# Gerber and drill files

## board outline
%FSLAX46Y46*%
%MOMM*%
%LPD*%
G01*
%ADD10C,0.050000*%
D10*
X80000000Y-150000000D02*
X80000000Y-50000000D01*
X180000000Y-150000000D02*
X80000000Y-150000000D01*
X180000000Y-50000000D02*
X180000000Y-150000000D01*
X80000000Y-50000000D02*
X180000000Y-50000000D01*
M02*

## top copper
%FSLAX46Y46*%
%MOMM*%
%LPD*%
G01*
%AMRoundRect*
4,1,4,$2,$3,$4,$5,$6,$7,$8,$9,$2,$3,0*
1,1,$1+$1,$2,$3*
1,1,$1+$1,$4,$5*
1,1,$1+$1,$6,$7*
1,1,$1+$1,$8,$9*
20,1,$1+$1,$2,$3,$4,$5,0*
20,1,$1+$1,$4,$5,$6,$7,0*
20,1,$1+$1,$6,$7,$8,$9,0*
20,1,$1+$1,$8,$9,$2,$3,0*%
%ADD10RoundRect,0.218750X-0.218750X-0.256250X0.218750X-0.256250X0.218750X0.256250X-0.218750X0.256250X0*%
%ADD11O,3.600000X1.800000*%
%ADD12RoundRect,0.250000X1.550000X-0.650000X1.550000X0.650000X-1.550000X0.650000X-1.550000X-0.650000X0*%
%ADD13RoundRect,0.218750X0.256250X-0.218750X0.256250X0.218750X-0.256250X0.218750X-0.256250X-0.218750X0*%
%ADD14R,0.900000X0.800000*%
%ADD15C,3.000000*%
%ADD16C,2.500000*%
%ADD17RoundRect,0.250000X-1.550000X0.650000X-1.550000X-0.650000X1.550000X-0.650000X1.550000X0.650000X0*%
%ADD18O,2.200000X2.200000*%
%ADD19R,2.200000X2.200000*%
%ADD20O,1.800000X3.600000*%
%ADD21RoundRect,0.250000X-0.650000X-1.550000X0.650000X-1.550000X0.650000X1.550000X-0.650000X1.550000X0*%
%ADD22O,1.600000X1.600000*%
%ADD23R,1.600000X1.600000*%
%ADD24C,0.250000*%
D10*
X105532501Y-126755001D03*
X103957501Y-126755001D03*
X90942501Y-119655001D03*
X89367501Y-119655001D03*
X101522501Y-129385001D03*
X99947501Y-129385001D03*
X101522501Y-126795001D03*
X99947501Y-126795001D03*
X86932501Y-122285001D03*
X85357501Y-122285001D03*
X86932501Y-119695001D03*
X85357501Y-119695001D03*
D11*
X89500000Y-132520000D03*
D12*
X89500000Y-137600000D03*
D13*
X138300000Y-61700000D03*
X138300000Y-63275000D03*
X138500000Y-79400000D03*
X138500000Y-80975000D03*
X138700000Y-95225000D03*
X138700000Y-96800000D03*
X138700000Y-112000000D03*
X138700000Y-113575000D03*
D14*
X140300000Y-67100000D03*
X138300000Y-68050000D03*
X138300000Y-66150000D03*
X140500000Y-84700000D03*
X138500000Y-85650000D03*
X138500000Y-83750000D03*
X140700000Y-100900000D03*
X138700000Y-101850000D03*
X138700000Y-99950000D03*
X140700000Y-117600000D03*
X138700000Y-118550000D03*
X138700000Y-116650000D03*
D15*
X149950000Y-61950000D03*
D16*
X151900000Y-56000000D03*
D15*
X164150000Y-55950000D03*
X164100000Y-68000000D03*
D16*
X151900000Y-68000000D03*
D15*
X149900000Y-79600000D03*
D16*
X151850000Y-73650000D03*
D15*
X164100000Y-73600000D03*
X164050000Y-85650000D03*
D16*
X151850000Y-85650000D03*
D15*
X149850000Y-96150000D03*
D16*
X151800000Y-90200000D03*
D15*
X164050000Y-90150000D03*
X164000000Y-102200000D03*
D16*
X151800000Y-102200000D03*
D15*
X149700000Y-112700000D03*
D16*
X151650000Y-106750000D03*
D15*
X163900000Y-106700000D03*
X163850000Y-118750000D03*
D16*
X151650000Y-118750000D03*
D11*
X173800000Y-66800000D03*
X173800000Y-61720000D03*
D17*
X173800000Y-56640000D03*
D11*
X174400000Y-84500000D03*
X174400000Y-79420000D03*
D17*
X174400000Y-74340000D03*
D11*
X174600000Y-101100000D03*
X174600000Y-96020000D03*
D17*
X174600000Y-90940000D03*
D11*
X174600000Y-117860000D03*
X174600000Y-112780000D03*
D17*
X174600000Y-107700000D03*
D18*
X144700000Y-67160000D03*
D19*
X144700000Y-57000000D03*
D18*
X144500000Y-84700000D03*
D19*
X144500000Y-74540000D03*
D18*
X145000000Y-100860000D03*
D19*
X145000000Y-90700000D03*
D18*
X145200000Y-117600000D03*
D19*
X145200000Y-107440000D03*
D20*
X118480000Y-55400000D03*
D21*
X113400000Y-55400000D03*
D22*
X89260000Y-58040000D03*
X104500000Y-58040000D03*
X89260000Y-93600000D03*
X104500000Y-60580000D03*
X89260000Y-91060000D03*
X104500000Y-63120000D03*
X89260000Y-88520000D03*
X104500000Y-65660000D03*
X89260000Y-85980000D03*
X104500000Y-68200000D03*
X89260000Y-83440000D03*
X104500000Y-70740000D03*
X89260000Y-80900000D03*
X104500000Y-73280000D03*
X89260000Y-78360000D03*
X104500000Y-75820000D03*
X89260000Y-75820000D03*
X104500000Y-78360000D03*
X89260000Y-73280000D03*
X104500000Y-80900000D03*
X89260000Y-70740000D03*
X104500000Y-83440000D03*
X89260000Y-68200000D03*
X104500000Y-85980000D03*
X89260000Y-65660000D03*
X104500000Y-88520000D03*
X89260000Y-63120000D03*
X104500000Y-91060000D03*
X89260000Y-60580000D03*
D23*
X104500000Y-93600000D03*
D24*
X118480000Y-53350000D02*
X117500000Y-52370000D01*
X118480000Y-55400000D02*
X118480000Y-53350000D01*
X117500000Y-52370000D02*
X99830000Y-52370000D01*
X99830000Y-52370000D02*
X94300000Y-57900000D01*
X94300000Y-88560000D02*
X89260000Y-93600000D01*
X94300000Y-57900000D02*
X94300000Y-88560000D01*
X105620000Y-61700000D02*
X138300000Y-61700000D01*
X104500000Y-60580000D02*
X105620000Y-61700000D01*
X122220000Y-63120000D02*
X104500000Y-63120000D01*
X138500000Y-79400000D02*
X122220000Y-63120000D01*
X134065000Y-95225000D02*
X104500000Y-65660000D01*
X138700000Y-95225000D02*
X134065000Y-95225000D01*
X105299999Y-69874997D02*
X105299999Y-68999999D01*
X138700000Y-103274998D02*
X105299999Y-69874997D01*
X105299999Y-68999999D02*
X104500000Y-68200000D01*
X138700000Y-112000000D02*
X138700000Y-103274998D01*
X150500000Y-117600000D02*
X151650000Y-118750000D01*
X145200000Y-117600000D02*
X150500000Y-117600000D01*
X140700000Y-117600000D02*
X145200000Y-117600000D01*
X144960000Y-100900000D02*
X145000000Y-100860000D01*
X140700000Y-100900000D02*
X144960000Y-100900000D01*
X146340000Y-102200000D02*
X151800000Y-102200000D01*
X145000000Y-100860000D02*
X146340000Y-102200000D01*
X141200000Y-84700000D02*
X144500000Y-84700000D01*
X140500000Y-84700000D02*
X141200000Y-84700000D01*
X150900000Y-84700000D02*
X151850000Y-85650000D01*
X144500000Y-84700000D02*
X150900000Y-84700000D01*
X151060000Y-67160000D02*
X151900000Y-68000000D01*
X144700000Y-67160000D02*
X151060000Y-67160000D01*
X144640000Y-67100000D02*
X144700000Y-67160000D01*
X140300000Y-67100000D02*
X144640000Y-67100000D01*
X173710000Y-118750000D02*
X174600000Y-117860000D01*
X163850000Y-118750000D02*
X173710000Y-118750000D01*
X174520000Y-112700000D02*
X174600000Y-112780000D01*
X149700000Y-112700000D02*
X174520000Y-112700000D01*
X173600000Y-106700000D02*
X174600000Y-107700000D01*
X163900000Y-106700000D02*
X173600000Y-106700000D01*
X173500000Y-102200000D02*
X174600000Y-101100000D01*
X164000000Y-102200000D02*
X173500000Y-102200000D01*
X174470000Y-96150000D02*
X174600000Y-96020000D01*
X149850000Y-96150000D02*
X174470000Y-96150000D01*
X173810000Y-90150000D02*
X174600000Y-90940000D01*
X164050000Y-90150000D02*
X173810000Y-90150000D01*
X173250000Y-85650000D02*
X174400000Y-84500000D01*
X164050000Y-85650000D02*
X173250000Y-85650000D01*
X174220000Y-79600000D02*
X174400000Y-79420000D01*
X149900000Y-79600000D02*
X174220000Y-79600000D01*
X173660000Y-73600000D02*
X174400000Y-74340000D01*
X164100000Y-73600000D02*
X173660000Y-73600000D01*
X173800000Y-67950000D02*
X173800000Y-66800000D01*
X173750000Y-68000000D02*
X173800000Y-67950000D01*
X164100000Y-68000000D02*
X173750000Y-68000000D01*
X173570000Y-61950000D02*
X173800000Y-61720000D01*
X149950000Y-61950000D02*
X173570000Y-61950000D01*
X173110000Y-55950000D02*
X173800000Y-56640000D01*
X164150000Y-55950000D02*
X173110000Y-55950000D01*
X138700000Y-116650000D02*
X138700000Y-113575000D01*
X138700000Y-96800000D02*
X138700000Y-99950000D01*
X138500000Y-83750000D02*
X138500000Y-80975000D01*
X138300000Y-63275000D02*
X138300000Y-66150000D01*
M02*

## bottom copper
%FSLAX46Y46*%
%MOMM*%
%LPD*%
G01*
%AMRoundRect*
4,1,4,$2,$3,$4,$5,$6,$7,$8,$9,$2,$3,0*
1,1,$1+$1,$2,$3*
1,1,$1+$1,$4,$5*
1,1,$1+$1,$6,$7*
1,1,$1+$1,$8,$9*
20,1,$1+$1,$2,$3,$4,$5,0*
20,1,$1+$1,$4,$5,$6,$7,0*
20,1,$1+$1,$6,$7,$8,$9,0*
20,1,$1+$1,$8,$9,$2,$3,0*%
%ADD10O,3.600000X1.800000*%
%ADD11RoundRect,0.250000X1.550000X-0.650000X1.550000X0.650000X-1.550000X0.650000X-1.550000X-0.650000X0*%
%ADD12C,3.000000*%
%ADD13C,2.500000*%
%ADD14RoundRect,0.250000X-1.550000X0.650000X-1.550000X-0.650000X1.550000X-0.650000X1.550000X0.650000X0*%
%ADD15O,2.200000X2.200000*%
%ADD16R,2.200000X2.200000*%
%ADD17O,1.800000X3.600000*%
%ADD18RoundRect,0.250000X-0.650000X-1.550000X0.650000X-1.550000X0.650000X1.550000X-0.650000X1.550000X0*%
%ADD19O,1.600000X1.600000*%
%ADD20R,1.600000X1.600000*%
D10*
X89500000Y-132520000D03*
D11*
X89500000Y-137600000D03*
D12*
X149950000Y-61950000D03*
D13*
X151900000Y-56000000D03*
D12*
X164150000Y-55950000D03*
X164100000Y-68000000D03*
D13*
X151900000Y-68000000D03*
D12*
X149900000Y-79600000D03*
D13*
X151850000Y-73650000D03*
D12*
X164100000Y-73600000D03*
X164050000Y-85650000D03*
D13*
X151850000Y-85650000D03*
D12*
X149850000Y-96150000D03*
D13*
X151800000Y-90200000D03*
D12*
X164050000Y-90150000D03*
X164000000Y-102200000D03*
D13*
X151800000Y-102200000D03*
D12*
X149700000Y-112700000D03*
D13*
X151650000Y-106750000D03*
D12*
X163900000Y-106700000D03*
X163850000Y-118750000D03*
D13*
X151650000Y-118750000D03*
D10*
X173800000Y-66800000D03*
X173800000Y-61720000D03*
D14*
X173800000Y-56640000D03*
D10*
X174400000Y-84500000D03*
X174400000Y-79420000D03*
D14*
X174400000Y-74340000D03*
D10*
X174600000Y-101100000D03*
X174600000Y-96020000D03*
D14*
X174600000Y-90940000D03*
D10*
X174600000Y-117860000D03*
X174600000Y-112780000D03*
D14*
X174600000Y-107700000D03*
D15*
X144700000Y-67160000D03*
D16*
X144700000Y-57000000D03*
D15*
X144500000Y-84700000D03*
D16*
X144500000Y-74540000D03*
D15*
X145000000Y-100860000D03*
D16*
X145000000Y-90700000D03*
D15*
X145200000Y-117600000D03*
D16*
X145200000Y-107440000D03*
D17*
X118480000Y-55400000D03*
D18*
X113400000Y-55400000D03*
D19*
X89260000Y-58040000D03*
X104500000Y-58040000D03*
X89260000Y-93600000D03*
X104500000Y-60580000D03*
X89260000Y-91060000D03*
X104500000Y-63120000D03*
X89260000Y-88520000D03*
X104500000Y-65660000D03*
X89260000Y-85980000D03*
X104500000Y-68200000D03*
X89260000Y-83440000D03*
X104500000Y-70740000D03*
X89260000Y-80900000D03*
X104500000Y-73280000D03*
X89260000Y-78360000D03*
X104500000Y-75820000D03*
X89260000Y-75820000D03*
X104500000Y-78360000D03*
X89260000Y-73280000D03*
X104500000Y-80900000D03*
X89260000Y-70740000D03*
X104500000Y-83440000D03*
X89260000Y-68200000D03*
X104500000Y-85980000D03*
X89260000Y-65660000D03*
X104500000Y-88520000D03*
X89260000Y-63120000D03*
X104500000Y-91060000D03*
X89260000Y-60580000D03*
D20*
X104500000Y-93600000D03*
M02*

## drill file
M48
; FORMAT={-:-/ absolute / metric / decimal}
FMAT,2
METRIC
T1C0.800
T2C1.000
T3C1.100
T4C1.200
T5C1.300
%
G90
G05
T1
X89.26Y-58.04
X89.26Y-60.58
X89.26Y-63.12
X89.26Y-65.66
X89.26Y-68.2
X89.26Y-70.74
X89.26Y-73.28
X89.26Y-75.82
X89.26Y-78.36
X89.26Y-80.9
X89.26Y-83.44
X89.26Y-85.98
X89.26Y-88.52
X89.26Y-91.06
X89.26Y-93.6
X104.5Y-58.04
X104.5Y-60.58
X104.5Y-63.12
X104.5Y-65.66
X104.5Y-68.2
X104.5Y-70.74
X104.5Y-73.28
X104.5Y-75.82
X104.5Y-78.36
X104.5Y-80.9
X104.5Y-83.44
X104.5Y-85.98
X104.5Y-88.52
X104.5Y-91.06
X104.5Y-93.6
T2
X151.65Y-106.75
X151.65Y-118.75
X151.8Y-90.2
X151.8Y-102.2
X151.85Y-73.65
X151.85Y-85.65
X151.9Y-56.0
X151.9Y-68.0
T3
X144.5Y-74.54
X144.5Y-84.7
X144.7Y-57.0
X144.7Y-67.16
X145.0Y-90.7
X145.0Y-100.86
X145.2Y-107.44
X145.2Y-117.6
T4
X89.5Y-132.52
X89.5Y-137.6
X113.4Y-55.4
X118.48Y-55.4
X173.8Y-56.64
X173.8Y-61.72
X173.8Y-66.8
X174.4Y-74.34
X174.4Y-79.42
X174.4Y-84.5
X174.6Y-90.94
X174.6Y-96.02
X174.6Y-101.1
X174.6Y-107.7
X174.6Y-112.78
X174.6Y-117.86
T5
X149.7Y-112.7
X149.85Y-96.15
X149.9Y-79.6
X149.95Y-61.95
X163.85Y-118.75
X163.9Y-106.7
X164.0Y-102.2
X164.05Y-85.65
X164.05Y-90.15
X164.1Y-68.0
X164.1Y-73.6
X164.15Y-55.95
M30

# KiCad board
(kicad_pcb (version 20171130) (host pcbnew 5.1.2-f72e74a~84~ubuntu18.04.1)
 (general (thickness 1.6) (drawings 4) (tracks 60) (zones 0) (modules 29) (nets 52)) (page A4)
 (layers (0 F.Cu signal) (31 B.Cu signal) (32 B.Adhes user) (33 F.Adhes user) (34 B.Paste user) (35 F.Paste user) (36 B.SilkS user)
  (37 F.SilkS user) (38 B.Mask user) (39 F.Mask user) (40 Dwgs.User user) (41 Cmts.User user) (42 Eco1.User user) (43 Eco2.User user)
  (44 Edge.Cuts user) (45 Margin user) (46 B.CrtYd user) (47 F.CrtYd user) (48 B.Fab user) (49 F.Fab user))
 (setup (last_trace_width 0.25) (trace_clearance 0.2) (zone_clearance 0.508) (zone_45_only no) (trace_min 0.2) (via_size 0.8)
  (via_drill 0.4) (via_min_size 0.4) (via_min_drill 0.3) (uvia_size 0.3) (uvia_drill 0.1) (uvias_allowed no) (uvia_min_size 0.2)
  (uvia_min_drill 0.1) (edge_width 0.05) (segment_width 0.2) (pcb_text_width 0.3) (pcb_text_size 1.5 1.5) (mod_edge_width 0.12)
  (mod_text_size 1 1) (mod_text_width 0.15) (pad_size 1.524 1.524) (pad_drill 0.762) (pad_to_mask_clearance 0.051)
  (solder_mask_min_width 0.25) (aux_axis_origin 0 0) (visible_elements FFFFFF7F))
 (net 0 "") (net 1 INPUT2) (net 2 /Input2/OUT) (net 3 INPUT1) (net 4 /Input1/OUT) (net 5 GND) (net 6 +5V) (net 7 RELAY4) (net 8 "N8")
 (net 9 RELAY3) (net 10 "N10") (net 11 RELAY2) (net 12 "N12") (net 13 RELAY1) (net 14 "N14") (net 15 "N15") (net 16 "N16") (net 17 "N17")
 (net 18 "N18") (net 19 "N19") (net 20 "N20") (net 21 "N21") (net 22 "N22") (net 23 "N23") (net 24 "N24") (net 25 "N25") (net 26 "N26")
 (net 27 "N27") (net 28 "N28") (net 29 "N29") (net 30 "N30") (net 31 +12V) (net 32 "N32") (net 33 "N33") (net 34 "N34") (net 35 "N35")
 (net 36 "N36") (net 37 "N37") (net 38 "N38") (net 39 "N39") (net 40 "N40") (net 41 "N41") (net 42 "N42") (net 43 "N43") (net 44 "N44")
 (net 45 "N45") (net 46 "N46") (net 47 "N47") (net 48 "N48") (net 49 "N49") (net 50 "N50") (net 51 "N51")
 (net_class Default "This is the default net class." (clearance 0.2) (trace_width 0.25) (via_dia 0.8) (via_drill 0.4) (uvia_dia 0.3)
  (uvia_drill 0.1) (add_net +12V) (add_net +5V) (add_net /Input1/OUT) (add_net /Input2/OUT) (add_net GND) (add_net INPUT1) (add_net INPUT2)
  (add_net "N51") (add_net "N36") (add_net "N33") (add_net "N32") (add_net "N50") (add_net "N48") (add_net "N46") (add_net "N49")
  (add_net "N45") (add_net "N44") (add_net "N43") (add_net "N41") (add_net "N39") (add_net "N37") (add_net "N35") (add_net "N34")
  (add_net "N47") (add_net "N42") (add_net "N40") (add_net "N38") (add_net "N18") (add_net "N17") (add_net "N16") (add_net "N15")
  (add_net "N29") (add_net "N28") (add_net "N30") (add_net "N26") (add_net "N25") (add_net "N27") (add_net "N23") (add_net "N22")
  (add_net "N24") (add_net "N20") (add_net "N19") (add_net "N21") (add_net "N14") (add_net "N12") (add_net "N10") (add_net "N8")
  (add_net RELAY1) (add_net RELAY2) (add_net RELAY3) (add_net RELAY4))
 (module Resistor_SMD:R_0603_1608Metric (layer F.Cu) (at 104.745001 126.755001)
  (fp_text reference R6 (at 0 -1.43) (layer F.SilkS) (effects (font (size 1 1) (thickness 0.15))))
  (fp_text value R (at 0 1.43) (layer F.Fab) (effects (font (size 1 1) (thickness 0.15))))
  (pad 2 smd roundrect (at 0.7875 0) (size 0.875 0.95) (layers F.Cu F.Paste F.Mask) (roundrect_rratio 0.25) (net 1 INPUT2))
  (pad 1 smd roundrect (at -0.7875 0) (size 0.875 0.95) (layers F.Cu F.Paste F.Mask) (roundrect_rratio 0.25) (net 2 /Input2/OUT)))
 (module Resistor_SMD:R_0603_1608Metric (layer F.Cu) (at 90.155001 119.655001)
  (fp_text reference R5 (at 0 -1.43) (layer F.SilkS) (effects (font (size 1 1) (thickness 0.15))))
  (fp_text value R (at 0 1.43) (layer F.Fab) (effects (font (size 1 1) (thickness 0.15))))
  (pad 2 smd roundrect (at 0.7875 0) (size 0.875 0.95) (layers F.Cu F.Paste F.Mask) (roundrect_rratio 0.25) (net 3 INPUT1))
  (pad 1 smd roundrect (at -0.7875 0) (size 0.875 0.95) (layers F.Cu F.Paste F.Mask) (roundrect_rratio 0.25) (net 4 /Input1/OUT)))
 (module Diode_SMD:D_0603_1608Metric (layer F.Cu) (at 100.735001 129.385001)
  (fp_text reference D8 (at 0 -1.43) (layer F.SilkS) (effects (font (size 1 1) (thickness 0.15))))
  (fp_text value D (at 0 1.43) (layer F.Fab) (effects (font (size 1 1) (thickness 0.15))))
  (pad 2 smd roundrect (at 0.7875 0) (size 0.875 0.95) (layers F.Cu F.Paste F.Mask) (roundrect_rratio 0.25) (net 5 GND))
  (pad 1 smd roundrect (at -0.7875 0) (size 0.875 0.95) (layers F.Cu F.Paste F.Mask) (roundrect_rratio 0.25) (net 2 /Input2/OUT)))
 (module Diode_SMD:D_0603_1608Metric (layer F.Cu) (at 100.735001 126.795001)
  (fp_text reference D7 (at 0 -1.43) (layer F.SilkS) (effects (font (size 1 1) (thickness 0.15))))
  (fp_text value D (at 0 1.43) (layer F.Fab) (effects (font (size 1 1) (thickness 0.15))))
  (pad 2 smd roundrect (at 0.7875 0) (size 0.875 0.95) (layers F.Cu F.Paste F.Mask) (roundrect_rratio 0.25) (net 2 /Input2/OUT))
  (pad 1 smd roundrect (at -0.7875 0) (size 0.875 0.95) (layers F.Cu F.Paste F.Mask) (roundrect_rratio 0.25) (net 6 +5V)))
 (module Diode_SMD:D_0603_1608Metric (layer F.Cu) (at 86.145001 122.285001)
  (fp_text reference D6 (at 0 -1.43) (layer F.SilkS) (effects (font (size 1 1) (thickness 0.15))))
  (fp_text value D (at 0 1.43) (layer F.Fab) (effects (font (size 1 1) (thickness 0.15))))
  (pad 2 smd roundrect (at 0.7875 0) (size 0.875 0.95) (layers F.Cu F.Paste F.Mask) (roundrect_rratio 0.25) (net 5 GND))
  (pad 1 smd roundrect (at -0.7875 0) (size 0.875 0.95) (layers F.Cu F.Paste F.Mask) (roundrect_rratio 0.25) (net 4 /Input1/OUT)))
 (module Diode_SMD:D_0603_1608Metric (layer F.Cu) (at 86.145001 119.695001)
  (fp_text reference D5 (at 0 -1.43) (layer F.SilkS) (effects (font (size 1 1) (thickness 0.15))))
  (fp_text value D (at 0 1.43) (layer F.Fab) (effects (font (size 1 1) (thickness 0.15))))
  (pad 2 smd roundrect (at 0.7875 0) (size 0.875 0.95) (layers F.Cu F.Paste F.Mask) (roundrect_rratio 0.25) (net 4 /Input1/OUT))
  (pad 1 smd roundrect (at -0.7875 0) (size 0.875 0.95) (layers F.Cu F.Paste F.Mask) (roundrect_rratio 0.25) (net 6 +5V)))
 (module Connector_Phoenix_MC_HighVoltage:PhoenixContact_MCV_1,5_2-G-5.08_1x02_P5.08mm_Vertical (layer F.Cu) (at 89.5 137.6 90)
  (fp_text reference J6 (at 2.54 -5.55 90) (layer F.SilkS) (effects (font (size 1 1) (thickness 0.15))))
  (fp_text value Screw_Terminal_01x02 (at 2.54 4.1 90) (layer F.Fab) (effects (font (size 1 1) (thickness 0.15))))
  (pad 2 thru_hole oval (at 5.08 0 90) (size 1.8 3.6) (drill 1.2) (layers *.Cu *.Mask) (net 3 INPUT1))
  (pad 1 thru_hole roundrect (at 0 0 90) (size 1.8 3.6) (drill 1.2) (layers *.Cu *.Mask) (roundrect_rratio 0.138889) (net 1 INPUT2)))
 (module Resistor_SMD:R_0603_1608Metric (layer F.Cu) (at 138.3 62.4875 90)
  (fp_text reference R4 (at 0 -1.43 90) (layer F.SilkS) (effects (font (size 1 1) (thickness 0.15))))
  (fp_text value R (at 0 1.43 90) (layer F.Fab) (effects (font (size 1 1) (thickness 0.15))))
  (pad 2 smd roundrect (at 0.7875 0 90) (size 0.875 0.95) (layers F.Cu F.Paste F.Mask) (roundrect_rratio 0.25) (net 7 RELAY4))
  (pad 1 smd roundrect (at -0.7875 0 90) (size 0.875 0.95) (layers F.Cu F.Paste F.Mask) (roundrect_rratio 0.25) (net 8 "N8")))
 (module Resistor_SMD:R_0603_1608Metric (layer F.Cu) (at 138.5 80.1875 90)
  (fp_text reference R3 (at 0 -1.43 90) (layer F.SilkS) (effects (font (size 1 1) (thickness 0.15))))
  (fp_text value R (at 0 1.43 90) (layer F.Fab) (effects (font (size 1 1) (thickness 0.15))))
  (pad 2 smd roundrect (at 0.7875 0 90) (size 0.875 0.95) (layers F.Cu F.Paste F.Mask) (roundrect_rratio 0.25) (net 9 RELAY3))
  (pad 1 smd roundrect (at -0.7875 0 90) (size 0.875 0.95) (layers F.Cu F.Paste F.Mask) (roundrect_rratio 0.25) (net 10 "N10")))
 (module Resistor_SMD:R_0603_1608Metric (layer F.Cu) (at 138.7 96.0125 90)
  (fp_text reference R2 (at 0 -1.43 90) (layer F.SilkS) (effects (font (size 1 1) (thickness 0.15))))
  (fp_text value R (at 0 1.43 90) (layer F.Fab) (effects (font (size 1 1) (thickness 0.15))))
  (pad 2 smd roundrect (at 0.7875 0 90) (size 0.875 0.95) (layers F.Cu F.Paste F.Mask) (roundrect_rratio 0.25) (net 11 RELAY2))
  (pad 1 smd roundrect (at -0.7875 0 90) (size 0.875 0.95) (layers F.Cu F.Paste F.Mask) (roundrect_rratio 0.25) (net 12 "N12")))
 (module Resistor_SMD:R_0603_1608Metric (layer F.Cu) (at 138.7 112.7875 90)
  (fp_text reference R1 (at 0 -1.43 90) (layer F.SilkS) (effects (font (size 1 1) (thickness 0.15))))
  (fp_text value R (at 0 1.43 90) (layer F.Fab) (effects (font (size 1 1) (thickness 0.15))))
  (pad 2 smd roundrect (at 0.7875 0 90) (size 0.875 0.95) (layers F.Cu F.Paste F.Mask) (roundrect_rratio 0.25) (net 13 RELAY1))
  (pad 1 smd roundrect (at -0.7875 0 90) (size 0.875 0.95) (layers F.Cu F.Paste F.Mask) (roundrect_rratio 0.25) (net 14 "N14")))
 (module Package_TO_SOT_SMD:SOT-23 (layer F.Cu) (at 139.3 67.1)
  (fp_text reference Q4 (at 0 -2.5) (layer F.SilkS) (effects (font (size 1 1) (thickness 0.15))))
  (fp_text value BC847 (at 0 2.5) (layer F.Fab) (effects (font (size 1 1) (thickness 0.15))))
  (pad 3 smd rect (at 1 0) (size 0.9 0.8) (layers F.Cu F.Paste F.Mask) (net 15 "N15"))
  (pad 2 smd rect (at -1 0.95) (size 0.9 0.8) (layers F.Cu F.Paste F.Mask) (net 5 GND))
  (pad 1 smd rect (at -1 -0.95) (size 0.9 0.8) (layers F.Cu F.Paste F.Mask) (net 8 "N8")))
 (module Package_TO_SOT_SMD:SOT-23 (layer F.Cu) (at 139.5 84.7)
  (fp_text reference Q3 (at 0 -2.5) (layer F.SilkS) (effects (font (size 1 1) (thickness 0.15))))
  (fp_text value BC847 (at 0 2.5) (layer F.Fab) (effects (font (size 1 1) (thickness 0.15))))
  (pad 3 smd rect (at 1 0) (size 0.9 0.8) (layers F.Cu F.Paste F.Mask) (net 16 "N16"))
  (pad 2 smd rect (at -1 0.95) (size 0.9 0.8) (layers F.Cu F.Paste F.Mask) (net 5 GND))
  (pad 1 smd rect (at -1 -0.95) (size 0.9 0.8) (layers F.Cu F.Paste F.Mask) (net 10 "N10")))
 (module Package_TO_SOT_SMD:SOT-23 (layer F.Cu) (at 139.7 100.9)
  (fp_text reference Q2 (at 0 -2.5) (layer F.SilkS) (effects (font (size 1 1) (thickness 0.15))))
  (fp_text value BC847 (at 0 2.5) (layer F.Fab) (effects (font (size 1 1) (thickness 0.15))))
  (pad 3 smd rect (at 1 0) (size 0.9 0.8) (layers F.Cu F.Paste F.Mask) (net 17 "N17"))
  (pad 2 smd rect (at -1 0.95) (size 0.9 0.8) (layers F.Cu F.Paste F.Mask) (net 5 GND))
  (pad 1 smd rect (at -1 -0.95) (size 0.9 0.8) (layers F.Cu F.Paste F.Mask) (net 12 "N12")))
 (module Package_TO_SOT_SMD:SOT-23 (layer F.Cu) (at 139.7 117.6)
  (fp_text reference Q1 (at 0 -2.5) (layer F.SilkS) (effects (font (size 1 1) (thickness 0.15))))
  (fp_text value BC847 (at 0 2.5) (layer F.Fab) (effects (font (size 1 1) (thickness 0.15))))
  (pad 3 smd rect (at 1 0) (size 0.9 0.8) (layers F.Cu F.Paste F.Mask) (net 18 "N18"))
  (pad 2 smd rect (at -1 0.95) (size 0.9 0.8) (layers F.Cu F.Paste F.Mask) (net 5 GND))
  (pad 1 smd rect (at -1 -0.95) (size 0.9 0.8) (layers F.Cu F.Paste F.Mask) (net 14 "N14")))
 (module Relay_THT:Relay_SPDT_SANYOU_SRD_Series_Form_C (layer F.Cu) (at 149.95 61.95)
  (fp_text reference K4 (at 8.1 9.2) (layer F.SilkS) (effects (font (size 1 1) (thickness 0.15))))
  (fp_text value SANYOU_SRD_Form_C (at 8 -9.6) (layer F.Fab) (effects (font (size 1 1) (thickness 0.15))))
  (pad 1 thru_hole circle (at 0 0 90) (size 3 3) (drill 1.3) (layers *.Cu *.Mask) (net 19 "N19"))
  (pad 5 thru_hole circle (at 1.95 -5.95 90) (size 2.5 2.5) (drill 1) (layers *.Cu *.Mask) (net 6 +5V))
  (pad 4 thru_hole circle (at 14.2 -6 90) (size 3 3) (drill 1.3) (layers *.Cu *.Mask) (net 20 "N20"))
  (pad 3 thru_hole circle (at 14.15 6.05 90) (size 3 3) (drill 1.3) (layers *.Cu *.Mask) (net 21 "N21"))
  (pad 2 thru_hole circle (at 1.95 6.05 90) (size 2.5 2.5) (drill 1) (layers *.Cu *.Mask) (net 15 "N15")))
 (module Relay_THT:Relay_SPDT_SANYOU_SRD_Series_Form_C (layer F.Cu) (at 149.9 79.6)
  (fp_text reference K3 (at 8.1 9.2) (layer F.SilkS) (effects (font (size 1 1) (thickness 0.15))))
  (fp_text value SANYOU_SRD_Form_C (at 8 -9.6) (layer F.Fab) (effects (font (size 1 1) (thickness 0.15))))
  (pad 1 thru_hole circle (at 0 0 90) (size 3 3) (drill 1.3) (layers *.Cu *.Mask) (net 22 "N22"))
  (pad 5 thru_hole circle (at 1.95 -5.95 90) (size 2.5 2.5) (drill 1) (layers *.Cu *.Mask) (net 6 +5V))
  (pad 4 thru_hole circle (at 14.2 -6 90) (size 3 3) (drill 1.3) (layers *.Cu *.Mask) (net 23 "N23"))
  (pad 3 thru_hole circle (at 14.15 6.05 90) (size 3 3) (drill 1.3) (layers *.Cu *.Mask) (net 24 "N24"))
  (pad 2 thru_hole circle (at 1.95 6.05 90) (size 2.5 2.5) (drill 1) (layers *.Cu *.Mask) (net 16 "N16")))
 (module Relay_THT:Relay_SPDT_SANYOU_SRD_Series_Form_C (layer F.Cu) (at 149.85 96.15)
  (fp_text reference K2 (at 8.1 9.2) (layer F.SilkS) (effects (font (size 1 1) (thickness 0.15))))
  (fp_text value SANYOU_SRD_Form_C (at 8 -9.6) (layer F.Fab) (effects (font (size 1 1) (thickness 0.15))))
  (pad 1 thru_hole circle (at 0 0 90) (size 3 3) (drill 1.3) (layers *.Cu *.Mask) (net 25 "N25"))
  (pad 5 thru_hole circle (at 1.95 -5.95 90) (size 2.5 2.5) (drill 1) (layers *.Cu *.Mask) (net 6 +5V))
  (pad 4 thru_hole circle (at 14.2 -6 90) (size 3 3) (drill 1.3) (layers *.Cu *.Mask) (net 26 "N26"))
  (pad 3 thru_hole circle (at 14.15 6.05 90) (size 3 3) (drill 1.3) (layers *.Cu *.Mask) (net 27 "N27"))
  (pad 2 thru_hole circle (at 1.95 6.05 90) (size 2.5 2.5) (drill 1) (layers *.Cu *.Mask) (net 17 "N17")))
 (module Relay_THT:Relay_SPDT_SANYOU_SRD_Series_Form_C (layer F.Cu) (at 149.7 112.7)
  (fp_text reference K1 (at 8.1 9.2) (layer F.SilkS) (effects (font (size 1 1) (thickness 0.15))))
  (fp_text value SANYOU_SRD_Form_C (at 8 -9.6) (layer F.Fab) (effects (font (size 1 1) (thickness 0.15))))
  (pad 1 thru_hole circle (at 0 0 90) (size 3 3) (drill 1.3) (layers *.Cu *.Mask) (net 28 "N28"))
  (pad 5 thru_hole circle (at 1.95 -5.95 90) (size 2.5 2.5) (drill 1) (layers *.Cu *.Mask) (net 6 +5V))
  (pad 4 thru_hole circle (at 14.2 -6 90) (size 3 3) (drill 1.3) (layers *.Cu *.Mask) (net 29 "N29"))
  (pad 3 thru_hole circle (at 14.15 6.05 90) (size 3 3) (drill 1.3) (layers *.Cu *.Mask) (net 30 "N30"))
  (pad 2 thru_hole circle (at 1.95 6.05 90) (size 2.5 2.5) (drill 1) (layers *.Cu *.Mask) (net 18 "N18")))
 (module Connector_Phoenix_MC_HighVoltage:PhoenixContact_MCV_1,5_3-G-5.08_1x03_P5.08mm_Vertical (layer F.Cu) (at 173.8 56.64 270)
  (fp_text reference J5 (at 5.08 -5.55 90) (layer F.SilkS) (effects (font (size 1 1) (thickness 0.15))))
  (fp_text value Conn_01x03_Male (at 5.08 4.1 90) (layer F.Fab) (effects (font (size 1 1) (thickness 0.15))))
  (pad 3 thru_hole oval (at 10.16 0 270) (size 1.8 3.6) (drill 1.2) (layers *.Cu *.Mask) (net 21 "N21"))
  (pad 2 thru_hole oval (at 5.08 0 270) (size 1.8 3.6) (drill 1.2) (layers *.Cu *.Mask) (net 19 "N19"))
  (pad 1 thru_hole roundrect (at 0 0 270) (size 1.8 3.6) (drill 1.2) (layers *.Cu *.Mask) (roundrect_rratio 0.138889) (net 20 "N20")))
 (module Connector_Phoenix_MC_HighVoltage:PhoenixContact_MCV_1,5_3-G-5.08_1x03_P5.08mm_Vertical (layer F.Cu) (at 174.4 74.34 270)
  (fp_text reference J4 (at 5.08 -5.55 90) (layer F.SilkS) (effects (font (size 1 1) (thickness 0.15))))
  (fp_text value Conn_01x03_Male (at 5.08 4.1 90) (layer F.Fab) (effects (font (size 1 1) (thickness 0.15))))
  (pad 3 thru_hole oval (at 10.16 0 270) (size 1.8 3.6) (drill 1.2) (layers *.Cu *.Mask) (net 24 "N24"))
  (pad 2 thru_hole oval (at 5.08 0 270) (size 1.8 3.6) (drill 1.2) (layers *.Cu *.Mask) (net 22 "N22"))
  (pad 1 thru_hole roundrect (at 0 0 270) (size 1.8 3.6) (drill 1.2) (layers *.Cu *.Mask) (roundrect_rratio 0.138889) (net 23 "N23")))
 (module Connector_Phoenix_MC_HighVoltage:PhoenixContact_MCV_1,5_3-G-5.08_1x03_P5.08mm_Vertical (layer F.Cu) (at 174.6 90.94 270)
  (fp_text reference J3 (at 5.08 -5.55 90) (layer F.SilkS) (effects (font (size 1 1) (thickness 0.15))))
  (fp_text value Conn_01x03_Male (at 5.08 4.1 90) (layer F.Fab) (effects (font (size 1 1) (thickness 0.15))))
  (pad 3 thru_hole oval (at 10.16 0 270) (size 1.8 3.6) (drill 1.2) (layers *.Cu *.Mask) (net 27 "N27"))
  (pad 2 thru_hole oval (at 5.08 0 270) (size 1.8 3.6) (drill 1.2) (layers *.Cu *.Mask) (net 25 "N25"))
  (pad 1 thru_hole roundrect (at 0 0 270) (size 1.8 3.6) (drill 1.2) (layers *.Cu *.Mask) (roundrect_rratio 0.138889) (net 26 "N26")))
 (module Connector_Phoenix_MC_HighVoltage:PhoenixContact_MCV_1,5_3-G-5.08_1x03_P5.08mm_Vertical (layer F.Cu) (at 174.6 107.7 270)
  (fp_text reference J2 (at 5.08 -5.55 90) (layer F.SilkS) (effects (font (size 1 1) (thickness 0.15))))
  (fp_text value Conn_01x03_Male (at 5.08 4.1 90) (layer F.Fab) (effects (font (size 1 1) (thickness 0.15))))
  (pad 3 thru_hole oval (at 10.16 0 270) (size 1.8 3.6) (drill 1.2) (layers *.Cu *.Mask) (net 30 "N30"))
  (pad 2 thru_hole oval (at 5.08 0 270) (size 1.8 3.6) (drill 1.2) (layers *.Cu *.Mask) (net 28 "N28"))
  (pad 1 thru_hole roundrect (at 0 0 270) (size 1.8 3.6) (drill 1.2) (layers *.Cu *.Mask) (roundrect_rratio 0.138889) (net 29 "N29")))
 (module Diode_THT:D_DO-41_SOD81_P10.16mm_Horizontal (layer F.Cu) (at 144.7 57 270)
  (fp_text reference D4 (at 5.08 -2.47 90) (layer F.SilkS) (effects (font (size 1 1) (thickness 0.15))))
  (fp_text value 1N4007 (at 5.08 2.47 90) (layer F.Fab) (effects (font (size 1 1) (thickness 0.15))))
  (pad 2 thru_hole oval (at 10.16 0 270) (size 2.2 2.2) (drill 1.1) (layers *.Cu *.Mask) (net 15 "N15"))
  (pad 1 thru_hole rect (at 0 0 270) (size 2.2 2.2) (drill 1.1) (layers *.Cu *.Mask) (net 6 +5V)))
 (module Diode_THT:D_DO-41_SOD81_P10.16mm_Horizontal (layer F.Cu) (at 144.5 74.54 270)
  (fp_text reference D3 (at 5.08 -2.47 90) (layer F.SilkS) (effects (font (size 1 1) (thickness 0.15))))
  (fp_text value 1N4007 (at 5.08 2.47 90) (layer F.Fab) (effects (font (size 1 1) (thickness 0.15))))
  (pad 2 thru_hole oval (at 10.16 0 270) (size 2.2 2.2) (drill 1.1) (layers *.Cu *.Mask) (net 16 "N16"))
  (pad 1 thru_hole rect (at 0 0 270) (size 2.2 2.2) (drill 1.1) (layers *.Cu *.Mask) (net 6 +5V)))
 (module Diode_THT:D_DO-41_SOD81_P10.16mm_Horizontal (layer F.Cu) (at 145 90.7 270)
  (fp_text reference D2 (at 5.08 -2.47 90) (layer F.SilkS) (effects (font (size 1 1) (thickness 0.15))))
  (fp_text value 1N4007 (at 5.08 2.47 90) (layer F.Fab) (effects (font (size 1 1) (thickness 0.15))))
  (pad 2 thru_hole oval (at 10.16 0 270) (size 2.2 2.2) (drill 1.1) (layers *.Cu *.Mask) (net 17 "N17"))
  (pad 1 thru_hole rect (at 0 0 270) (size 2.2 2.2) (drill 1.1) (layers *.Cu *.Mask) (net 6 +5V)))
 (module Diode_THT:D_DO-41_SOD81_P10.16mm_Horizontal (layer F.Cu) (at 145.2 107.44 270)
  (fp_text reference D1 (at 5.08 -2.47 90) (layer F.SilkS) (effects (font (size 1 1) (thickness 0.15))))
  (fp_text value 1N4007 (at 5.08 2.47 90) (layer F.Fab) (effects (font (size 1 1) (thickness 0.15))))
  (pad 2 thru_hole oval (at 10.16 0 270) (size 2.2 2.2) (drill 1.1) (layers *.Cu *.Mask) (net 18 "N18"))
  (pad 1 thru_hole rect (at 0 0 270) (size 2.2 2.2) (drill 1.1) (layers *.Cu *.Mask) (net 6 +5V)))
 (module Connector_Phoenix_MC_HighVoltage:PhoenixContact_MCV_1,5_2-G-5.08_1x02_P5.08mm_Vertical (layer F.Cu) (at 113.4 55.4)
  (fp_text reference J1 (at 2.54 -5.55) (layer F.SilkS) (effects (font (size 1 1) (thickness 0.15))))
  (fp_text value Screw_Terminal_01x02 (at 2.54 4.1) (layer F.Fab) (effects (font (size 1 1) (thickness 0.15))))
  (pad 2 thru_hole oval (at 5.08 0) (size 1.8 3.6) (drill 1.2) (layers *.Cu *.Mask) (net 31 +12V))
  (pad 1 thru_hole roundrect (at 0 0) (size 1.8 3.6) (drill 1.2) (layers *.Cu *.Mask) (roundrect_rratio 0.138889) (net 5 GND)))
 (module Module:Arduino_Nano (layer F.Cu) (at 104.5 93.6 180)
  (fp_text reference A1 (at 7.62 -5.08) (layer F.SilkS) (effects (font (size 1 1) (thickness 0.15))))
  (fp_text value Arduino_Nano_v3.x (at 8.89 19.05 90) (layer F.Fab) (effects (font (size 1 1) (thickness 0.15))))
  (pad 16 thru_hole oval (at 15.24 35.56 180) (size 1.6 1.6) (drill 0.8) (layers *.Cu *.Mask) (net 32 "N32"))
  (pad 15 thru_hole oval (at 0 35.56 180) (size 1.6 1.6) (drill 0.8) (layers *.Cu *.Mask) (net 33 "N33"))
  (pad 30 thru_hole oval (at 15.24 0 180) (size 1.6 1.6) (drill 0.8) (layers *.Cu *.Mask) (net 31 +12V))
  (pad 14 thru_hole oval (at 0 33.02 180) (size 1.6 1.6) (drill 0.8) (layers *.Cu *.Mask) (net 7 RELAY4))
  (pad 29 thru_hole oval (at 15.24 2.54 180) (size 1.6 1.6) (drill 0.8) (layers *.Cu *.Mask) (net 5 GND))
  (pad 13 thru_hole oval (at 0 30.48 180) (size 1.6 1.6) (drill 0.8) (layers *.Cu *.Mask) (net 9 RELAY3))
  (pad 28 thru_hole oval (at 15.24 5.08 180) (size 1.6 1.6) (drill 0.8) (layers *.Cu *.Mask) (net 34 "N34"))
  (pad 12 thru_hole oval (at 0 27.94 180) (size 1.6 1.6) (drill 0.8) (layers *.Cu *.Mask) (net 11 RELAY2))
  (pad 27 thru_hole oval (at 15.24 7.62 180) (size 1.6 1.6) (drill 0.8) (layers *.Cu *.Mask) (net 6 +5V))
  (pad 11 thru_hole oval (at 0 25.4 180) (size 1.6 1.6) (drill 0.8) (layers *.Cu *.Mask) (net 13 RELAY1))
  (pad 26 thru_hole oval (at 15.24 10.16 180) (size 1.6 1.6) (drill 0.8) (layers *.Cu *.Mask) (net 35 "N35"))
  (pad 10 thru_hole oval (at 0 22.86 180) (size 1.6 1.6) (drill 0.8) (layers *.Cu *.Mask) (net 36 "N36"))
  (pad 25 thru_hole oval (at 15.24 12.7 180) (size 1.6 1.6) (drill 0.8) (layers *.Cu *.Mask) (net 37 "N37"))
  (pad 9 thru_hole oval (at 0 20.32 180) (size 1.6 1.6) (drill 0.8) (layers *.Cu *.Mask) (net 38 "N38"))
  (pad 24 thru_hole oval (at 15.24 15.24 180) (size 1.6 1.6) (drill 0.8) (layers *.Cu *.Mask) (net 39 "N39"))
  (pad 8 thru_hole oval (at 0 17.78 180) (size 1.6 1.6) (drill 0.8) (layers *.Cu *.Mask) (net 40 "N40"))
  (pad 23 thru_hole oval (at 15.24 17.78 180) (size 1.6 1.6) (drill 0.8) (layers *.Cu *.Mask) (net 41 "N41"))
  (pad 7 thru_hole oval (at 0 15.24 180) (size 1.6 1.6) (drill 0.8) (layers *.Cu *.Mask) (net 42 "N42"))
  (pad 22 thru_hole oval (at 15.24 20.32 180) (size 1.6 1.6) (drill 0.8) (layers *.Cu *.Mask) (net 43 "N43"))
  (pad 6 thru_hole oval (at 0 12.7 180) (size 1.6 1.6) (drill 0.8) (layers *.Cu *.Mask) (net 2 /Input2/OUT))
  (pad 21 thru_hole oval (at 15.24 22.86 180) (size 1.6 1.6) (drill 0.8) (layers *.Cu *.Mask) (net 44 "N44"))
  (pad 5 thru_hole oval (at 0 10.16 180) (size 1.6 1.6) (drill 0.8) (layers *.Cu *.Mask) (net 4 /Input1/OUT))
  (pad 20 thru_hole oval (at 15.24 25.4 180) (size 1.6 1.6) (drill 0.8) (layers *.Cu *.Mask) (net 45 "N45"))
  (pad 4 thru_hole oval (at 0 7.62 180) (size 1.6 1.6) (drill 0.8) (layers *.Cu *.Mask) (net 5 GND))
  (pad 19 thru_hole oval (at 15.24 27.94 180) (size 1.6 1.6) (drill 0.8) (layers *.Cu *.Mask) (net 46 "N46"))
  (pad 3 thru_hole oval (at 0 5.08 180) (size 1.6 1.6) (drill 0.8) (layers *.Cu *.Mask) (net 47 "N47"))
  (pad 18 thru_hole oval (at 15.24 30.48 180) (size 1.6 1.6) (drill 0.8) (layers *.Cu *.Mask) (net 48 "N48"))
  (pad 2 thru_hole oval (at 0 2.54 180) (size 1.6 1.6) (drill 0.8) (layers *.Cu *.Mask) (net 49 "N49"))
  (pad 17 thru_hole oval (at 15.24 33.02 180) (size 1.6 1.6) (drill 0.8) (layers *.Cu *.Mask) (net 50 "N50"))
  (pad 1 thru_hole rect (at 0 0 180) (size 1.6 1.6) (drill 0.8) (layers *.Cu *.Mask) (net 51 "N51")))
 (gr_line (start 80 150) (end 80 50) (layer Edge.Cuts) (width 0.05))
 (gr_line (start 180 150) (end 80 150) (layer Edge.Cuts) (width 0.05))
 (gr_line (start 180 50) (end 180 150) (layer Edge.Cuts) (width 0.05))
 (gr_line (start 80 50) (end 180 50) (layer Edge.Cuts) (width 0.05))
 (segment (start 118.48 53.35) (end 117.5 52.37) (width 0.25) (layer F.Cu) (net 31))
 (segment (start 118.48 55.4) (end 118.48 53.35) (width 0.25) (layer F.Cu) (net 31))
 (segment (start 117.5 52.37) (end 99.83 52.37) (width 0.25) (layer F.Cu) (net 31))
 (segment (start 99.83 52.37) (end 94.3 57.9) (width 0.25) (layer F.Cu) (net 31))
 (segment (start 94.3 88.56) (end 89.26 93.6) (width 0.25) (layer F.Cu) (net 31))
 (segment (start 94.3 57.9) (end 94.3 88.56) (width 0.25) (layer F.Cu) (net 31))
 (segment (start 105.62 61.7) (end 138.3 61.7) (width 0.25) (layer F.Cu) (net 7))
 (segment (start 104.5 60.58) (end 105.62 61.7) (width 0.25) (layer F.Cu) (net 7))
 (segment (start 122.22 63.12) (end 104.5 63.12) (width 0.25) (layer F.Cu) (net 9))
 (segment (start 138.5 79.4) (end 122.22 63.12) (width 0.25) (layer F.Cu) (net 9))
 (segment (start 134.065 95.225) (end 104.5 65.66) (width 0.25) (layer F.Cu) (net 11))
 (segment (start 138.7 95.225) (end 134.065 95.225) (width 0.25) (layer F.Cu) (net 11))
 (segment (start 105.299999 69.874997) (end 105.299999 68.999999) (width 0.25) (layer F.Cu) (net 13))
 (segment (start 138.7 103.274998) (end 105.299999 69.874997) (width 0.25) (layer F.Cu) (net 13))
 (segment (start 105.299999 68.999999) (end 104.5 68.2) (width 0.25) (layer F.Cu) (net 13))
 (segment (start 138.7 112) (end 138.7 103.274998) (width 0.25) (layer F.Cu) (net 13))
 (segment (start 150.5 117.6) (end 151.65 118.75) (width 0.25) (layer F.Cu) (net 18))
 (segment (start 145.2 117.6) (end 150.5 117.6) (width 0.25) (layer F.Cu) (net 18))
 (segment (start 140.7 117.6) (end 145.2 117.6) (width 0.25) (layer F.Cu) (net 18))
 (segment (start 144.96 100.9) (end 145 100.86) (width 0.25) (layer F.Cu) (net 17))
 (segment (start 140.7 100.9) (end 144.96 100.9) (width 0.25) (layer F.Cu) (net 17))
 (segment (start 146.34 102.2) (end 151.8 102.2) (width 0.25) (layer F.Cu) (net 17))
 (segment (start 145 100.86) (end 146.34 102.2) (width 0.25) (layer F.Cu) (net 17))
 (segment (start 141.2 84.7) (end 144.5 84.7) (width 0.25) (layer F.Cu) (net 16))
 (segment (start 140.5 84.7) (end 141.2 84.7) (width 0.25) (layer F.Cu) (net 16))
 (segment (start 150.9 84.7) (end 151.85 85.65) (width 0.25) (layer F.Cu) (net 16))
 (segment (start 144.5 84.7) (end 150.9 84.7) (width 0.25) (layer F.Cu) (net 16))
 (segment (start 151.06 67.16) (end 151.9 68) (width 0.25) (layer F.Cu) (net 15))
 (segment (start 144.7 67.16) (end 151.06 67.16) (width 0.25) (layer F.Cu) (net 15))
 (segment (start 144.64 67.1) (end 144.7 67.16) (width 0.25) (layer F.Cu) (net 15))
 (segment (start 140.3 67.1) (end 144.64 67.1) (width 0.25) (layer F.Cu) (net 15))
 (segment (start 173.71 118.75) (end 174.6 117.86) (width 0.25) (layer F.Cu) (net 30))
 (segment (start 163.85 118.75) (end 173.71 118.75) (width 0.25) (layer F.Cu) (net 30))
 (segment (start 174.52 112.7) (end 174.6 112.78) (width 0.25) (layer F.Cu) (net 28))
 (segment (start 149.7 112.7) (end 174.52 112.7) (width 0.25) (layer F.Cu) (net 28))
 (segment (start 173.6 106.7) (end 174.6 107.7) (width 0.25) (layer F.Cu) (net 29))
 (segment (start 163.9 106.7) (end 173.6 106.7) (width 0.25) (layer F.Cu) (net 29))
 (segment (start 173.5 102.2) (end 174.6 101.1) (width 0.25) (layer F.Cu) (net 27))
 (segment (start 164 102.2) (end 173.5 102.2) (width 0.25) (layer F.Cu) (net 27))
 (segment (start 174.47 96.15) (end 174.6 96.02) (width 0.25) (layer F.Cu) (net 25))
 (segment (start 149.85 96.15) (end 174.47 96.15) (width 0.25) (layer F.Cu) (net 25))
 (segment (start 173.81 90.15) (end 174.6 90.94) (width 0.25) (layer F.Cu) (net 26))
 (segment (start 164.05 90.15) (end 173.81 90.15) (width 0.25) (layer F.Cu) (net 26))
 (segment (start 173.25 85.65) (end 174.4 84.5) (width 0.25) (layer F.Cu) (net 24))
 (segment (start 164.05 85.65) (end 173.25 85.65) (width 0.25) (layer F.Cu) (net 24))
 (segment (start 174.22 79.6) (end 174.4 79.42) (width 0.25) (layer F.Cu) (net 22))
 (segment (start 149.9 79.6) (end 174.22 79.6) (width 0.25) (layer F.Cu) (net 22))
 (segment (start 173.66 73.6) (end 174.4 74.34) (width 0.25) (layer F.Cu) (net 23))
 (segment (start 164.1 73.6) (end 173.66 73.6) (width 0.25) (layer F.Cu) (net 23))
 (segment (start 173.8 67.95) (end 173.8 66.8) (width 0.25) (layer F.Cu) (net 21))
 (segment (start 173.75 68) (end 173.8 67.95) (width 0.25) (layer F.Cu) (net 21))
 (segment (start 164.1 68) (end 173.75 68) (width 0.25) (layer F.Cu) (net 21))
 (segment (start 173.57 61.95) (end 173.8 61.72) (width 0.25) (layer F.Cu) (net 19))
 (segment (start 149.95 61.95) (end 173.57 61.95) (width 0.25) (layer F.Cu) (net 19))
 (segment (start 173.11 55.95) (end 173.8 56.64) (width 0.25) (layer F.Cu) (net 20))
 (segment (start 164.15 55.95) (end 173.11 55.95) (width 0.25) (layer F.Cu) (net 20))
 (segment (start 138.7 116.65) (end 138.7 113.575) (width 0.25) (layer F.Cu) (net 14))
 (segment (start 138.7 96.8) (end 138.7 99.95) (width 0.25) (layer F.Cu) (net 12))
 (segment (start 138.5 83.75) (end 138.5 80.975) (width 0.25) (layer F.Cu) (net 10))
 (segment (start 138.3 63.275) (end 138.3 66.15) (width 0.25) (layer F.Cu) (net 8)))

